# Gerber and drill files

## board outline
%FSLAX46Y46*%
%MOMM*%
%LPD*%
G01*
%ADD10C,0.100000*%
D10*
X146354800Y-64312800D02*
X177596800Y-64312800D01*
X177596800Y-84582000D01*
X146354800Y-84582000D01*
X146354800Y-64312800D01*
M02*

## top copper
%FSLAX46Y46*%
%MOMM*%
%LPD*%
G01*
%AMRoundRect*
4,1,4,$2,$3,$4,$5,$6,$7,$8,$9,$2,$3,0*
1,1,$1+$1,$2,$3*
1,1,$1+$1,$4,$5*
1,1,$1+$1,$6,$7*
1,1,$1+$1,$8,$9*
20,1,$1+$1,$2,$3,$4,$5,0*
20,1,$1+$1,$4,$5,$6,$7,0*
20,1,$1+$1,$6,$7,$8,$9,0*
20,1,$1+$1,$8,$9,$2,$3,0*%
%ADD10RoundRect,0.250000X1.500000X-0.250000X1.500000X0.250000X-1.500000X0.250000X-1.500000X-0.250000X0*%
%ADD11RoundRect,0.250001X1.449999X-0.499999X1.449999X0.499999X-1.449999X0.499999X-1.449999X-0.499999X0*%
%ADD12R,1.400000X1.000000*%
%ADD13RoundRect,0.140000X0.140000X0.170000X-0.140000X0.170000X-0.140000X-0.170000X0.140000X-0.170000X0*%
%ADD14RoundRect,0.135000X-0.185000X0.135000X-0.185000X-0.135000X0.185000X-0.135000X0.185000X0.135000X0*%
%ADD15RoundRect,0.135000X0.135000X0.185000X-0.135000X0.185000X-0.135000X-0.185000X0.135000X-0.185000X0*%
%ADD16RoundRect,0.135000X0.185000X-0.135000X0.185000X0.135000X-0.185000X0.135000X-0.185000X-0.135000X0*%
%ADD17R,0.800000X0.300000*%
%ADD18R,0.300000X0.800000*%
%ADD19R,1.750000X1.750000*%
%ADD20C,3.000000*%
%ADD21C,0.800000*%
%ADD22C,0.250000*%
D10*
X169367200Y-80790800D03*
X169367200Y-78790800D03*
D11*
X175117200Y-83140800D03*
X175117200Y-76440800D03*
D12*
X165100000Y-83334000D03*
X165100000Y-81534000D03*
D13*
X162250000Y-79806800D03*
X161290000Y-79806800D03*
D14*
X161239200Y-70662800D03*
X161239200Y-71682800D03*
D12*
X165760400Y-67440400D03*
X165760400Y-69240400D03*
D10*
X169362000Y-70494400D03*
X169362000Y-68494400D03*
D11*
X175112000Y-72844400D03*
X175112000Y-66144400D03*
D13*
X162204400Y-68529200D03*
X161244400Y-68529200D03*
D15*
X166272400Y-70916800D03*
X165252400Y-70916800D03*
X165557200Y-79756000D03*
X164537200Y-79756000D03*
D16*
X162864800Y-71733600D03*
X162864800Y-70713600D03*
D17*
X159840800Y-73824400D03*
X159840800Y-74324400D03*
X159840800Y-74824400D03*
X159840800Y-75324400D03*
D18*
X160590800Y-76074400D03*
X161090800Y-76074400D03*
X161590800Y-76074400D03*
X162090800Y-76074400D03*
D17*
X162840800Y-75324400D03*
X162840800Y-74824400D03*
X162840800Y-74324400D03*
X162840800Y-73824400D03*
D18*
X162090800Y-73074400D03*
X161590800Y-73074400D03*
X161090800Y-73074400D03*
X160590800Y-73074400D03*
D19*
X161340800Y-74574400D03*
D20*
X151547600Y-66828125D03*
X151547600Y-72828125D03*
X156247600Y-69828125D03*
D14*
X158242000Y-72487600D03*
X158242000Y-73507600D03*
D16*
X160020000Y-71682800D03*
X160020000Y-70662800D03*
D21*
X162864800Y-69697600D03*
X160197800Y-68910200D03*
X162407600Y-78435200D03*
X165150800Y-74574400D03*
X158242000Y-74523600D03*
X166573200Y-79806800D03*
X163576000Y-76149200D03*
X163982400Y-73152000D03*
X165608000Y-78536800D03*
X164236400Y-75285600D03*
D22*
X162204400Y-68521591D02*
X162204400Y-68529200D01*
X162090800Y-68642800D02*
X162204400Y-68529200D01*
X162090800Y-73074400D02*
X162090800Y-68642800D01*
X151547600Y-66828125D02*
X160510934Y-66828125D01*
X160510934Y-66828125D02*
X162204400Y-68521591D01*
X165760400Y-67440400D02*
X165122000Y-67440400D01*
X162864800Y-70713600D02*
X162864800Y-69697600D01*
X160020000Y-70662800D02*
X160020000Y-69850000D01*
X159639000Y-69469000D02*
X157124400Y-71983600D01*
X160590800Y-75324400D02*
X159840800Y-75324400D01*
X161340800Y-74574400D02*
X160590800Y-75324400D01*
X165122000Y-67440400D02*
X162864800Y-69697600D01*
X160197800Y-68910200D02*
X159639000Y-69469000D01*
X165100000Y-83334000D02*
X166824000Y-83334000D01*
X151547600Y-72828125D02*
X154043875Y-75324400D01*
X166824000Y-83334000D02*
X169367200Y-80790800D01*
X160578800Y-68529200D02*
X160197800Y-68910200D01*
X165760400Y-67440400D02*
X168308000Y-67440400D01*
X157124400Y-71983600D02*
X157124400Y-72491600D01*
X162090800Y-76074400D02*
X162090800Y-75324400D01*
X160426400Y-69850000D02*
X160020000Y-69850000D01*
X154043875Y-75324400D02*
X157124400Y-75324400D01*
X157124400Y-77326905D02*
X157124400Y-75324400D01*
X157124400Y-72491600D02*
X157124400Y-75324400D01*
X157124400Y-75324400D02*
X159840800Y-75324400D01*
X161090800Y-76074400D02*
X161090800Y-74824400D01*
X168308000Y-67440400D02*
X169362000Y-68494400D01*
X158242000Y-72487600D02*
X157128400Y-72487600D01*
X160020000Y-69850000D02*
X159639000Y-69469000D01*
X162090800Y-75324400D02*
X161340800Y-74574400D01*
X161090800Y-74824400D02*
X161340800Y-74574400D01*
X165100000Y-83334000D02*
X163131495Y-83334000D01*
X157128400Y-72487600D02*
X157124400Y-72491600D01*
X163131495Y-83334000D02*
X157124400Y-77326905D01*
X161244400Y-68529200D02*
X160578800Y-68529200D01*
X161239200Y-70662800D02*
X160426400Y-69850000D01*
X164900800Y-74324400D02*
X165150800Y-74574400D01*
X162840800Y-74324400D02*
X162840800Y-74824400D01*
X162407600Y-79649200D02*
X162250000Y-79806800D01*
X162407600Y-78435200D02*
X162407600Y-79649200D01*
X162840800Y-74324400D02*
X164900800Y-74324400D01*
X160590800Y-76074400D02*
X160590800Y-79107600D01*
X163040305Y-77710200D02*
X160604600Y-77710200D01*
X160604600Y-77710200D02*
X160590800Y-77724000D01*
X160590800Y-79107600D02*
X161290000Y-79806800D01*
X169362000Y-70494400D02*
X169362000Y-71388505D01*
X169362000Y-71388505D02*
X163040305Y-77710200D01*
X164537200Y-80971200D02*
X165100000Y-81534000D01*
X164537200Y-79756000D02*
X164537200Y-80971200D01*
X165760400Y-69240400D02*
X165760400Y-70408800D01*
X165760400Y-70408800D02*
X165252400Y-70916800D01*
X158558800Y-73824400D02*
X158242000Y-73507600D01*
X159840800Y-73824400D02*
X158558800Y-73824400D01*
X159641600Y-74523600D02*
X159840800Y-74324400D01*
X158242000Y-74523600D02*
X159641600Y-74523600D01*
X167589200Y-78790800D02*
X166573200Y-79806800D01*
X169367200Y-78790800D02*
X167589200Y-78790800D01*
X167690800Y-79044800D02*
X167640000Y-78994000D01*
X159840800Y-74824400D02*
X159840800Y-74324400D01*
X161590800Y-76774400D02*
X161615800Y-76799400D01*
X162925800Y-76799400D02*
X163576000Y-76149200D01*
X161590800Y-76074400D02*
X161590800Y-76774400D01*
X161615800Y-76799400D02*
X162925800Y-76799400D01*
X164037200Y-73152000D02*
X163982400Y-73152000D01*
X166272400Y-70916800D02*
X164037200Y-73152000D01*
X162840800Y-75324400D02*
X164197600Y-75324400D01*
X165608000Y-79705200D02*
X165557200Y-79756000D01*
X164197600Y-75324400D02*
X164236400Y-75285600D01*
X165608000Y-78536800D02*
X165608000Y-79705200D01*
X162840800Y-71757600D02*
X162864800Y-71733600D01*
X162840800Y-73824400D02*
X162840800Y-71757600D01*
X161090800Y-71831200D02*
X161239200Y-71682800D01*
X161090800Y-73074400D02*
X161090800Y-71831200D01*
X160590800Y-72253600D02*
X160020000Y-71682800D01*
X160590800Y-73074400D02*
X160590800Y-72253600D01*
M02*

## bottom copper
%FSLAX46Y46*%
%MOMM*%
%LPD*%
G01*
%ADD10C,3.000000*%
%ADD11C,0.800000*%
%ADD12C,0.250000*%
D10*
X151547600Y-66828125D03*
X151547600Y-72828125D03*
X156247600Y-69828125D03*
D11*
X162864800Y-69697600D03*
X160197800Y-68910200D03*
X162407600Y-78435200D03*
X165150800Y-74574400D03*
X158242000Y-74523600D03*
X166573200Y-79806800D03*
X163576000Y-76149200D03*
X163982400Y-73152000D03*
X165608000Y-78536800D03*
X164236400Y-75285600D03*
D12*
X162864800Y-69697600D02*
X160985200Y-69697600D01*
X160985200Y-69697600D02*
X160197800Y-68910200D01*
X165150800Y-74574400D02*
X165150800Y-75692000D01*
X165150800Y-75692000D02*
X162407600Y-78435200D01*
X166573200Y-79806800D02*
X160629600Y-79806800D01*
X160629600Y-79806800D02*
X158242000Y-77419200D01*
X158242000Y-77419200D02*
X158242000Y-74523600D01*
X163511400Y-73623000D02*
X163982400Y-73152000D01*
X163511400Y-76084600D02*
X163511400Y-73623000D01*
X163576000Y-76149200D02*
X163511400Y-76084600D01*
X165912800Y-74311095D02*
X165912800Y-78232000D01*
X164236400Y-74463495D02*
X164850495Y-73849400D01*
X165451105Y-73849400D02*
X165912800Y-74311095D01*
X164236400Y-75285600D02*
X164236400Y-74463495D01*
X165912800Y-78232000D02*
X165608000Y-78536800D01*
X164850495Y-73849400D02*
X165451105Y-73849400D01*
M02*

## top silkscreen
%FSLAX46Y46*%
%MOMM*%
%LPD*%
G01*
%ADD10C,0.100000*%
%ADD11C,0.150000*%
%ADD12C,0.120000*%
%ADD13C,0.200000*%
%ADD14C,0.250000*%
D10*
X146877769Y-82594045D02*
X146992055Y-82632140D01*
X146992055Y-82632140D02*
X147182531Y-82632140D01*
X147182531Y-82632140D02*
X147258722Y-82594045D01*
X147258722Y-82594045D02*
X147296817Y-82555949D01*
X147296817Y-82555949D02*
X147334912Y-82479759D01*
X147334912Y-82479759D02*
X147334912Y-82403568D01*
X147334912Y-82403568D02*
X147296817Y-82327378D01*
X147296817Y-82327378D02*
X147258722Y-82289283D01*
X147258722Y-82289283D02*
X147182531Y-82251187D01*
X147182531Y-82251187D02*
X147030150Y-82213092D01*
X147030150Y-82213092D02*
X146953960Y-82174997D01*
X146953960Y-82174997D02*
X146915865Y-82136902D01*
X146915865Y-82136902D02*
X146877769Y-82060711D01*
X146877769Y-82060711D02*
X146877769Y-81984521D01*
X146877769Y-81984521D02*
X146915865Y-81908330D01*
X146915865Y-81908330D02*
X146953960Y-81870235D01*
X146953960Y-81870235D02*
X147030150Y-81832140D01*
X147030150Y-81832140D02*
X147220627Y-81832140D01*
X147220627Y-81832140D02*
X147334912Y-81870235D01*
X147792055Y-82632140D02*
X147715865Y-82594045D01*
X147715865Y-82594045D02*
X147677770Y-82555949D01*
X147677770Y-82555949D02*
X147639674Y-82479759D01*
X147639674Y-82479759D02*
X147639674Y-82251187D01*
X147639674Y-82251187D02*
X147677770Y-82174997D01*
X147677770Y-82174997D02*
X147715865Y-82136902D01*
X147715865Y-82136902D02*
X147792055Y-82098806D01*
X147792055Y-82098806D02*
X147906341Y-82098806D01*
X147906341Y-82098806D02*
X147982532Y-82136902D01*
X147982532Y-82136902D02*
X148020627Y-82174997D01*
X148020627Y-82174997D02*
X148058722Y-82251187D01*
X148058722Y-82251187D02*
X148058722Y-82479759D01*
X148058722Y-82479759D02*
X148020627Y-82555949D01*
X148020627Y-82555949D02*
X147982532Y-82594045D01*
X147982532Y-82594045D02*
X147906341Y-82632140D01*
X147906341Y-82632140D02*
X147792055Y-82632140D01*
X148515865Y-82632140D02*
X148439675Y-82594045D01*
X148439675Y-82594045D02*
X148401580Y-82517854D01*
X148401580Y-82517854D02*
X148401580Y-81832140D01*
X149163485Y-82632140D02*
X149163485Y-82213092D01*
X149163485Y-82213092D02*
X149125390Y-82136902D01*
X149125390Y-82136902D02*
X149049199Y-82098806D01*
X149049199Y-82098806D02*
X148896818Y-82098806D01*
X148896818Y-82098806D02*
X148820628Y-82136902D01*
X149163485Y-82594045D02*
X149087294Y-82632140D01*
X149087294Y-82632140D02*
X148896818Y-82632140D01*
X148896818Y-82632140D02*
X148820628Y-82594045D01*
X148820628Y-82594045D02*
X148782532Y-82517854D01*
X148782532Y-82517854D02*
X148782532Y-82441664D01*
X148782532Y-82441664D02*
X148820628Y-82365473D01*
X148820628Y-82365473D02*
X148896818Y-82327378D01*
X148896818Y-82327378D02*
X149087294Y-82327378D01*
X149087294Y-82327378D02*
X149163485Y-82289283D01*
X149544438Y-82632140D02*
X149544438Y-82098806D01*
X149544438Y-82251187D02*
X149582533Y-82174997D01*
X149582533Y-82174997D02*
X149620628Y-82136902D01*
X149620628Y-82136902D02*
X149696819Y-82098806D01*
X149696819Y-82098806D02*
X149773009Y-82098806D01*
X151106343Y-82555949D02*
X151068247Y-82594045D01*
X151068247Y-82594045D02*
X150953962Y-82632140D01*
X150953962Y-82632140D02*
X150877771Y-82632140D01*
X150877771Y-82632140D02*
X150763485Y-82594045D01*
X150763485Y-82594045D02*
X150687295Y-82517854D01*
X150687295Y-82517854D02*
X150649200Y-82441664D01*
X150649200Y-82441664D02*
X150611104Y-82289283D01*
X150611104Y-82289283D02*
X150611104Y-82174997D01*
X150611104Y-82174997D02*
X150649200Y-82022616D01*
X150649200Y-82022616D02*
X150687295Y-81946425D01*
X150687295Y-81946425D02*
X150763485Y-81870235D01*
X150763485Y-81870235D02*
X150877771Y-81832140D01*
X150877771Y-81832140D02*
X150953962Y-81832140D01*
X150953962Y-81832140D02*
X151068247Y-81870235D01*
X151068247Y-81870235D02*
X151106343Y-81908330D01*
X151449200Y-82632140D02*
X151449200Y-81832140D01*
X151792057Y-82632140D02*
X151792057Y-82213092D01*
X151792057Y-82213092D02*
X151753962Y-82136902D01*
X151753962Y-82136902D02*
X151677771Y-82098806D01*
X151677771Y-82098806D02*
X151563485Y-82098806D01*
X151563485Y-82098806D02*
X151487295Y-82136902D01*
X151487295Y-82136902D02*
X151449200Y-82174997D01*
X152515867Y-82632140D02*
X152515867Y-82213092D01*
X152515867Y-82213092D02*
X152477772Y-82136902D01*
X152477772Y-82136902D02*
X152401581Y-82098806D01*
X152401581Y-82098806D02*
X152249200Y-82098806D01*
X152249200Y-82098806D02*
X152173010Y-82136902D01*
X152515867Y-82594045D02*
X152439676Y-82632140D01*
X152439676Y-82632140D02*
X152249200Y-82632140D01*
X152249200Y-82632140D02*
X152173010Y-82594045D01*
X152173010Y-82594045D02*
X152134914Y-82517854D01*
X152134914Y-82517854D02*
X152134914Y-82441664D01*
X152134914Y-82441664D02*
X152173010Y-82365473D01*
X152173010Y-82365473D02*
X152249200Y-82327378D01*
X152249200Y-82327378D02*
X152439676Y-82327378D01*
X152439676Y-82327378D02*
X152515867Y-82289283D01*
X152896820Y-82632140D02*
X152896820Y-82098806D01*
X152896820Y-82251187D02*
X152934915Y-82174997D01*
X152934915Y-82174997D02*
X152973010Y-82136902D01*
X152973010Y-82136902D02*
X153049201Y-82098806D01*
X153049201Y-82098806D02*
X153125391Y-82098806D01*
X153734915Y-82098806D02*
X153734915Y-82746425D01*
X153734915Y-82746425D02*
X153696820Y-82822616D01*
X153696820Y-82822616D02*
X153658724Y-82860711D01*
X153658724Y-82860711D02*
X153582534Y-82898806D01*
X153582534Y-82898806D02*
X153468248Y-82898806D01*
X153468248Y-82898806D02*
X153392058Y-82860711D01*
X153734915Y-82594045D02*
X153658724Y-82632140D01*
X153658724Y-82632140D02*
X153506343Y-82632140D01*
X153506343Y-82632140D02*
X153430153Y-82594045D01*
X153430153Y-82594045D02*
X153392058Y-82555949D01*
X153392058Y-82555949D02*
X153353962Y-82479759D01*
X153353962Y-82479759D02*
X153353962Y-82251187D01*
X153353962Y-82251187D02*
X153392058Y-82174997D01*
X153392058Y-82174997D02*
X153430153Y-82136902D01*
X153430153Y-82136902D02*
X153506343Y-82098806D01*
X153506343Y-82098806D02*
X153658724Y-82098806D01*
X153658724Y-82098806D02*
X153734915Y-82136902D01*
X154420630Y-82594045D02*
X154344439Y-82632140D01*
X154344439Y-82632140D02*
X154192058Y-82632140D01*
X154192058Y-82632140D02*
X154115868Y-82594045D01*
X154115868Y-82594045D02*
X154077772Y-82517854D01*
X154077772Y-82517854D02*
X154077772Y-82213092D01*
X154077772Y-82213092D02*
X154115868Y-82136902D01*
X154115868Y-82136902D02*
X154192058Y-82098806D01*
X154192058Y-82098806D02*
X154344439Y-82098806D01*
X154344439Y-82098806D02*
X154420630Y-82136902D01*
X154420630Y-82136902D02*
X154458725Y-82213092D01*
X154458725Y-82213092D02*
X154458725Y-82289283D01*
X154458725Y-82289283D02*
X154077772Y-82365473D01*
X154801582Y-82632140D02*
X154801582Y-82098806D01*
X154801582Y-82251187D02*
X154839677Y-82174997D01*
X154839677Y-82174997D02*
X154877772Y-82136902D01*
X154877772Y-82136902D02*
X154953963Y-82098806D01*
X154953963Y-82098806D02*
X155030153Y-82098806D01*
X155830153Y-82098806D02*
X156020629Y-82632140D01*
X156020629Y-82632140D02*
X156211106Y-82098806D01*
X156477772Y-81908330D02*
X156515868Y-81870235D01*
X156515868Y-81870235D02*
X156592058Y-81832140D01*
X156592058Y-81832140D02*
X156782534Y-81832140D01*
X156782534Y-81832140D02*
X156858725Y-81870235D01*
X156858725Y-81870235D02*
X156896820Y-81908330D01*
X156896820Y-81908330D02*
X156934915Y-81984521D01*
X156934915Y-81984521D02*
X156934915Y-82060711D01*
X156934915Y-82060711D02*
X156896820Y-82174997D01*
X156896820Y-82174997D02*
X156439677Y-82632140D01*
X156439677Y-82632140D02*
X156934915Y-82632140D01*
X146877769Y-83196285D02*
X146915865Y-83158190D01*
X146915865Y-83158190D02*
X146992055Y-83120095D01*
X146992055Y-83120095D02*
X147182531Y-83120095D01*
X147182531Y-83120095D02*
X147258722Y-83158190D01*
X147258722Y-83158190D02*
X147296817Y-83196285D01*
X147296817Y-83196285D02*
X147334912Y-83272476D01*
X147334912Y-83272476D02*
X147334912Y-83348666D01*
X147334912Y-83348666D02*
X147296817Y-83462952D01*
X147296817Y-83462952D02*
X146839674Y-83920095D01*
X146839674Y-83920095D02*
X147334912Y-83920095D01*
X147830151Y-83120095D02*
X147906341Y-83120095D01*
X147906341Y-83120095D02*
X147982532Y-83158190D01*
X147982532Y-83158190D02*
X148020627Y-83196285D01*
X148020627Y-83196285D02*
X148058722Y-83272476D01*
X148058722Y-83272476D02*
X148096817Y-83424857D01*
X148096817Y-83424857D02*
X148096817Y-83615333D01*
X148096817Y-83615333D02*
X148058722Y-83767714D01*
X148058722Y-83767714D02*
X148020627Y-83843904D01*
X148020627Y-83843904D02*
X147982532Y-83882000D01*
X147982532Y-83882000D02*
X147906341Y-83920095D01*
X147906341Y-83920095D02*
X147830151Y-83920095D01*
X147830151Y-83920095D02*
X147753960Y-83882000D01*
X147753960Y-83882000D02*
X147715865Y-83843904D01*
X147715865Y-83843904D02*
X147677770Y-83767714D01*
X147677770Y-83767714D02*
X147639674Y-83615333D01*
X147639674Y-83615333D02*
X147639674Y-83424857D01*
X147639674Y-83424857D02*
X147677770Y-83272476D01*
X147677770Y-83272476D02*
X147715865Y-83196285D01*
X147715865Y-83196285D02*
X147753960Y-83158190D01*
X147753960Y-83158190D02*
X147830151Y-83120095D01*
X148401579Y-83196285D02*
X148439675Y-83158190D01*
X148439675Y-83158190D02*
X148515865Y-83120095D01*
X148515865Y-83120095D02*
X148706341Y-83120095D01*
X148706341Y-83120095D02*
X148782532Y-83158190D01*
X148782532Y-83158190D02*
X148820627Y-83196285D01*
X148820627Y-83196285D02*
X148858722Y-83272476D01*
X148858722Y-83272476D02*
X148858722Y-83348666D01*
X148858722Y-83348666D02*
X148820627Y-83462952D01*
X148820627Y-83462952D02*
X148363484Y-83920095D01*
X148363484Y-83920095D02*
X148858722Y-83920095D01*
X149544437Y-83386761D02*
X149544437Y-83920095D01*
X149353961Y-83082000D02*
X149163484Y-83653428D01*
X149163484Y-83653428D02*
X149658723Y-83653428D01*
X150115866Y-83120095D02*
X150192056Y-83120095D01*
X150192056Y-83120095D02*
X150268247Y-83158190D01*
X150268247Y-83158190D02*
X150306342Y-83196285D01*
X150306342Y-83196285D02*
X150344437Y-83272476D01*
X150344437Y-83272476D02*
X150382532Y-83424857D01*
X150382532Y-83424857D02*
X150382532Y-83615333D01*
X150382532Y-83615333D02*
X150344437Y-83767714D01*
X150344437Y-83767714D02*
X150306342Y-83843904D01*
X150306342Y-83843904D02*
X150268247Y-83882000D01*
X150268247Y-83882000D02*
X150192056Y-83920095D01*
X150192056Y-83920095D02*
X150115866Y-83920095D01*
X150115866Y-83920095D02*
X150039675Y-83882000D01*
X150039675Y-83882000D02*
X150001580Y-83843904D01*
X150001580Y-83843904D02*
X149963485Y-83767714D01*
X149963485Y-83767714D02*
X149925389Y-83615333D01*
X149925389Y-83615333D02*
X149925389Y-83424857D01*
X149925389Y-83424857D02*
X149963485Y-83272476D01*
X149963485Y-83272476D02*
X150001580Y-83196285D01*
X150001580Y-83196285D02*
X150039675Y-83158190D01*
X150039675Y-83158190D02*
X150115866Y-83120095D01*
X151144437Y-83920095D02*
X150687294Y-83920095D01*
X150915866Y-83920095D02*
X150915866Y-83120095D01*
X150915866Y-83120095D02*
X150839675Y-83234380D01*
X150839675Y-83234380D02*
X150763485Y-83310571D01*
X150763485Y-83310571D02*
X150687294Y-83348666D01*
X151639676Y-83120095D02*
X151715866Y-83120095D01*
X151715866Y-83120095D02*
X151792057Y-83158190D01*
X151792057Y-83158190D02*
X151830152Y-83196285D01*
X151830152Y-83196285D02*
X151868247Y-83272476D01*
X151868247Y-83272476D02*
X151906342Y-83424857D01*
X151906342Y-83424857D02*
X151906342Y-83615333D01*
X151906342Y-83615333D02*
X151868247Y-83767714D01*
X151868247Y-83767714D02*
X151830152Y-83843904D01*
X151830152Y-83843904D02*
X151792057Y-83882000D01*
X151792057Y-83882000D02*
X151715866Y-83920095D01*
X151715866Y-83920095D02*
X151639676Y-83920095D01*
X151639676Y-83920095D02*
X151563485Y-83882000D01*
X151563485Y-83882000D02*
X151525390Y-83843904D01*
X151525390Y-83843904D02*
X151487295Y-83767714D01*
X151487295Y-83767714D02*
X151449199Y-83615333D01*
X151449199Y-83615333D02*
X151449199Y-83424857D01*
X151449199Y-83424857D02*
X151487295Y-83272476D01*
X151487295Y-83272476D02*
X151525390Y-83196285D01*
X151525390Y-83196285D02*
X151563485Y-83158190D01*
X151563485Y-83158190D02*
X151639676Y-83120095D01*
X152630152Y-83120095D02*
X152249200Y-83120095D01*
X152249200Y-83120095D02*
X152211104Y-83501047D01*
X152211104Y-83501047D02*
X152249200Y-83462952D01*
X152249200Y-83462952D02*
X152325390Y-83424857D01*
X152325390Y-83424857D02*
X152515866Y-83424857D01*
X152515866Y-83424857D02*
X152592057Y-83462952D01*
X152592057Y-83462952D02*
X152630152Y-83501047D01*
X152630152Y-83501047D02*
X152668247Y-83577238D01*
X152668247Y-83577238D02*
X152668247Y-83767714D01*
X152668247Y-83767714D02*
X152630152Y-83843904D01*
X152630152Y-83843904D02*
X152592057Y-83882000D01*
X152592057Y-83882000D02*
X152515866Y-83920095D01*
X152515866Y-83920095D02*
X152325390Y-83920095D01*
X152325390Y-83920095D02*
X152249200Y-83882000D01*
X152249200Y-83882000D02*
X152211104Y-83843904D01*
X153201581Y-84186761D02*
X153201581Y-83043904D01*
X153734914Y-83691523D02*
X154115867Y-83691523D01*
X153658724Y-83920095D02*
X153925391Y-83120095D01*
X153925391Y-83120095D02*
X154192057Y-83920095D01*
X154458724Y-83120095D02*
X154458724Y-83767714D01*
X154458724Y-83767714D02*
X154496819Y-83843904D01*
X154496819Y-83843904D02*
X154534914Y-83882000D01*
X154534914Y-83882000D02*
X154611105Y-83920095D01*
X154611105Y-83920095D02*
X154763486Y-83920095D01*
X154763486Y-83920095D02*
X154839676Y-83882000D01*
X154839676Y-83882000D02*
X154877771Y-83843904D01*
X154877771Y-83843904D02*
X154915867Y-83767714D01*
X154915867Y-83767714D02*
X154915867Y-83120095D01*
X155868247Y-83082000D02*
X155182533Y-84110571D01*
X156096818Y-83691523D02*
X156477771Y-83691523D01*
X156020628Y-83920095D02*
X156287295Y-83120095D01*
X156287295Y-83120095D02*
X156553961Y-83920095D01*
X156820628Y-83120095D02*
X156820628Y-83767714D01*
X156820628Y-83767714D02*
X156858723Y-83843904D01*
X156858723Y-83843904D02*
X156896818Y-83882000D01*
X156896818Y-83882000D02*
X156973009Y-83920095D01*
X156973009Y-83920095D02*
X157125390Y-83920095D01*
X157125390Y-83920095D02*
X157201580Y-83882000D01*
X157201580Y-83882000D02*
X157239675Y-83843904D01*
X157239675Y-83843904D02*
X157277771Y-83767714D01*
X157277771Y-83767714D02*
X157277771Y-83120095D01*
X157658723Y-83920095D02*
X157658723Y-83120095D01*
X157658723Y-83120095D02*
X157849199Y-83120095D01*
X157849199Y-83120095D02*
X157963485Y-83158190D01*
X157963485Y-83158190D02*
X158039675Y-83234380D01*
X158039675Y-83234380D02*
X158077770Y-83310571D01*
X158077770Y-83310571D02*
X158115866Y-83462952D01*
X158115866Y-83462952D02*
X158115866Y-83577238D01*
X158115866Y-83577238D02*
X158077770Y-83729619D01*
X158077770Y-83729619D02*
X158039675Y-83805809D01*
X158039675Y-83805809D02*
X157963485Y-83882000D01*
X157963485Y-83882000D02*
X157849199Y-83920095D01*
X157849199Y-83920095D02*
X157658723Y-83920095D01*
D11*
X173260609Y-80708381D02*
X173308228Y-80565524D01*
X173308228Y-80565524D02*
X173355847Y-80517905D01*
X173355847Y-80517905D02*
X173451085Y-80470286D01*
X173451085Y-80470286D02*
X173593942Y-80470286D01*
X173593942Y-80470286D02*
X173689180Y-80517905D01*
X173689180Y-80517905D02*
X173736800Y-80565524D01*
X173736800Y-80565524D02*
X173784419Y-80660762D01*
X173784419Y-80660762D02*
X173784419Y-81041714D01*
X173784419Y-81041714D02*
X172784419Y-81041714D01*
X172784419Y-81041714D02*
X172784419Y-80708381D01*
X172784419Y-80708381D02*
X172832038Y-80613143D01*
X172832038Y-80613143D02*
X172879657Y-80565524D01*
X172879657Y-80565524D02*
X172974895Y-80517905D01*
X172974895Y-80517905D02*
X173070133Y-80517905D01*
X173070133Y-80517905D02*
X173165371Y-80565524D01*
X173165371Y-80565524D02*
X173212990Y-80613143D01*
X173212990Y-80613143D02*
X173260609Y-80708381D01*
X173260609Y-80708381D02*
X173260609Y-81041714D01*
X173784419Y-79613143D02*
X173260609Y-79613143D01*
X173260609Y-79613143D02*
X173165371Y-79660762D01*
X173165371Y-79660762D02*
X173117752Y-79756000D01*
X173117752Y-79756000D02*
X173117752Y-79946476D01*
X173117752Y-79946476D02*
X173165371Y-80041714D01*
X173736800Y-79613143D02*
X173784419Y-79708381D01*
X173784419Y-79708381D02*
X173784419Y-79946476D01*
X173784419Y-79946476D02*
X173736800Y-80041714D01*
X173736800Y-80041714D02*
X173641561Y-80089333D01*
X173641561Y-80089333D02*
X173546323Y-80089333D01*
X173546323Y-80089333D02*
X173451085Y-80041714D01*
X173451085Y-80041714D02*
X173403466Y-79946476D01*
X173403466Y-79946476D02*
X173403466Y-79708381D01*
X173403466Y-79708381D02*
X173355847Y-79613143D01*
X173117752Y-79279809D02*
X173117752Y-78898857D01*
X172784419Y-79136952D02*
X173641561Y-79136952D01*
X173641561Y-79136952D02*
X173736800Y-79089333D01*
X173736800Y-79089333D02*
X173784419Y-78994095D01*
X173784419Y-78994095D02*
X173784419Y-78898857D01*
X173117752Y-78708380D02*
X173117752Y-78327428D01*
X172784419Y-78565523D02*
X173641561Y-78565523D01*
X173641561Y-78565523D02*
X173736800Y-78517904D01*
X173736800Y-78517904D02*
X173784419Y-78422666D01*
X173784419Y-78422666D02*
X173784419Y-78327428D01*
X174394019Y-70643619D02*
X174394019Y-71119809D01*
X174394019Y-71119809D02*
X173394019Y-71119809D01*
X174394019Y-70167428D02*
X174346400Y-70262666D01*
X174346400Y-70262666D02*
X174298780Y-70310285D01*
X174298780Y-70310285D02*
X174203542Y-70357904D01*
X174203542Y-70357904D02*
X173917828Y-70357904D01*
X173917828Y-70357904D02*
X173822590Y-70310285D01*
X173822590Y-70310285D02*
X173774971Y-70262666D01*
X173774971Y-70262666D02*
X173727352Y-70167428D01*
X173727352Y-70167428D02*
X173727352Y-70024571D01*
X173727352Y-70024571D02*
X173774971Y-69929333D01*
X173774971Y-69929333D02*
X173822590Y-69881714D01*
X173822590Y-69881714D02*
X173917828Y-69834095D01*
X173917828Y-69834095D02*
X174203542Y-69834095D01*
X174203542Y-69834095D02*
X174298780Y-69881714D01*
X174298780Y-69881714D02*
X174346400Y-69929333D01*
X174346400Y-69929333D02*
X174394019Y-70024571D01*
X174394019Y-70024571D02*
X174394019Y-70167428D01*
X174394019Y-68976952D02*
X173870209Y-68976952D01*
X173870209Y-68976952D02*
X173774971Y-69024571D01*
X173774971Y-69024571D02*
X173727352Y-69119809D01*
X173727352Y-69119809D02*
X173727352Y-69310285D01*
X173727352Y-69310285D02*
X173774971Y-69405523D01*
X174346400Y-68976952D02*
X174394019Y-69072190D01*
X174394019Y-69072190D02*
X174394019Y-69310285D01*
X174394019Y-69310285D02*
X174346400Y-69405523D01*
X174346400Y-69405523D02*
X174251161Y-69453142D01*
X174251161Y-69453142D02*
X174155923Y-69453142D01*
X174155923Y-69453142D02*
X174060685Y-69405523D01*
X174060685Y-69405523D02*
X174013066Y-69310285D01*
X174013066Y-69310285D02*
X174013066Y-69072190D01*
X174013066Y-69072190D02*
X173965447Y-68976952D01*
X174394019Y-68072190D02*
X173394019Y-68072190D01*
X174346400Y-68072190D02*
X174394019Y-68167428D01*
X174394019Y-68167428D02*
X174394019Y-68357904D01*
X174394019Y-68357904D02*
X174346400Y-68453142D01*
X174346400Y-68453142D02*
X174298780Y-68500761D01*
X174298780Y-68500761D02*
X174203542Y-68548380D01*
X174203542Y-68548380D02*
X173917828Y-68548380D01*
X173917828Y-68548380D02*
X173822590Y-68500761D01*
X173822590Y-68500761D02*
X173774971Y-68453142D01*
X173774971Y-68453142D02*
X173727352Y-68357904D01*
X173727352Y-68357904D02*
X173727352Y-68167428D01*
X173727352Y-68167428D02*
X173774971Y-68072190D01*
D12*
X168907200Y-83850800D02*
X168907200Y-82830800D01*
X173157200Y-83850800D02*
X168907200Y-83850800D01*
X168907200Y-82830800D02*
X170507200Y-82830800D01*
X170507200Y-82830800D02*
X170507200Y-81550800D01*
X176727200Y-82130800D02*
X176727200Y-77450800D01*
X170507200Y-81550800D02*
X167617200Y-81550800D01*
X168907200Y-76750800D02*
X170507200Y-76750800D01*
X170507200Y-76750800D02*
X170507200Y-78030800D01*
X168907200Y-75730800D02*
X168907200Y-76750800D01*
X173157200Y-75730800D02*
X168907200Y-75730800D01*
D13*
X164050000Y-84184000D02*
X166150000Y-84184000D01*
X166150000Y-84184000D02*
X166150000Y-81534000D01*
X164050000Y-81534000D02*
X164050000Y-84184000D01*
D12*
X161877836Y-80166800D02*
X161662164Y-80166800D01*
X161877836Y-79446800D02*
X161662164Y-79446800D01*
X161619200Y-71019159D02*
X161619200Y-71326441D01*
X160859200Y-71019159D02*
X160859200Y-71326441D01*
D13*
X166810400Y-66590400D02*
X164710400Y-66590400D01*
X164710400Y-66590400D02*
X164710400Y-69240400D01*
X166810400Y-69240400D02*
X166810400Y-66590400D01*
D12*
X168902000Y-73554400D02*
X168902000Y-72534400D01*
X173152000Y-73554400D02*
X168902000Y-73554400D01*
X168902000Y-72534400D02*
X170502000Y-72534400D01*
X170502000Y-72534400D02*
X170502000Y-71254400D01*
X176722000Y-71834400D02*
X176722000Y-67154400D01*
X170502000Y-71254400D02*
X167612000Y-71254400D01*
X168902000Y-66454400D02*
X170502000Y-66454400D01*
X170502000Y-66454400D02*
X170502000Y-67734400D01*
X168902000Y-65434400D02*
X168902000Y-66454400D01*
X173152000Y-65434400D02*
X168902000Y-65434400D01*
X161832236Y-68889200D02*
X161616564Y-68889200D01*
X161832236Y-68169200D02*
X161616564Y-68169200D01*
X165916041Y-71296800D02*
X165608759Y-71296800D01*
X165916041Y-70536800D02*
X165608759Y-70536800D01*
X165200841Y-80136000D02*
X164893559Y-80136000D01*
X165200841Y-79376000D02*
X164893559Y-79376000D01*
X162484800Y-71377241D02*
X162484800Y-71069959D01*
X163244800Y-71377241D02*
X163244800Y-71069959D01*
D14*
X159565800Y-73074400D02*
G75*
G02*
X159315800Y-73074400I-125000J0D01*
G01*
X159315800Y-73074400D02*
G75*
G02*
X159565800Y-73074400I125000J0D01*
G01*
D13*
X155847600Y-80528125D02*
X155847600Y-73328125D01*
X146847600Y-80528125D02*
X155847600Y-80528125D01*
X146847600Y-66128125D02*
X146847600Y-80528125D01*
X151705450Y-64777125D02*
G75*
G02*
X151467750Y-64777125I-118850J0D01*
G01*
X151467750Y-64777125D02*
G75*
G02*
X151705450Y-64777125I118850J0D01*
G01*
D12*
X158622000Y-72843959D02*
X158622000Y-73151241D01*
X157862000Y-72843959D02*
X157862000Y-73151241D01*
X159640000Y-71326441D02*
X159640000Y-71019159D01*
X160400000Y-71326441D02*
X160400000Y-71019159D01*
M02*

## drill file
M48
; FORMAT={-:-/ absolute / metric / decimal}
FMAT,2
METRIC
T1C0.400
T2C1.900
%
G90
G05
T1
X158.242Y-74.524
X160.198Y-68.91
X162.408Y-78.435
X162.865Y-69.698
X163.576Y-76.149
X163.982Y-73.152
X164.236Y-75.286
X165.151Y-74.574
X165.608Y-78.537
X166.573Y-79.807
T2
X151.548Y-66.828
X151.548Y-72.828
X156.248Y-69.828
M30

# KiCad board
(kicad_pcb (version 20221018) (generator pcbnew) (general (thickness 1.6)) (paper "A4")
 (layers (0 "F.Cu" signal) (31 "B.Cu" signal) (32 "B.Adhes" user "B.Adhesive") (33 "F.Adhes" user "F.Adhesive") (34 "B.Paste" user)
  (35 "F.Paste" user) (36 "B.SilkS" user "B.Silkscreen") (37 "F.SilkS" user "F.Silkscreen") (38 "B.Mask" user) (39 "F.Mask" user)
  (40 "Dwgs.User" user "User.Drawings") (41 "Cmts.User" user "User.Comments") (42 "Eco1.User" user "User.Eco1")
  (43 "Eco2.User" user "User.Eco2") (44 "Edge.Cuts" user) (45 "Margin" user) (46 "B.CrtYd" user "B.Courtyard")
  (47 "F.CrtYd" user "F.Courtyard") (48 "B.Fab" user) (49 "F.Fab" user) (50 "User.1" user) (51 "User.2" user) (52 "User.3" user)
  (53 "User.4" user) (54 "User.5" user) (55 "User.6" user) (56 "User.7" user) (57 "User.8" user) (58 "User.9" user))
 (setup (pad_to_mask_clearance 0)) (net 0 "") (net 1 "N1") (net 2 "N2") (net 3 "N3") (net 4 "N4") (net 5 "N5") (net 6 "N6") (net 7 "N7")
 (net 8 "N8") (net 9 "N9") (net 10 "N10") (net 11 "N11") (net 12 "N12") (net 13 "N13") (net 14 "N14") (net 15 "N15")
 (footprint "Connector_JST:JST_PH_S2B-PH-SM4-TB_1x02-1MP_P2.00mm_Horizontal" (layer "F.Cu") (at 172.2172 79.7908 90)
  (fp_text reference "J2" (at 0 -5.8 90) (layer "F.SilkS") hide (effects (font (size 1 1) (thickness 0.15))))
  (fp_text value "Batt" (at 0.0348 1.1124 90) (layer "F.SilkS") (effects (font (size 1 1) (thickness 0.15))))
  (fp_line (start -4.06 -3.31) (end -3.04 -3.31) (stroke (width 0.12) (type solid)) (layer "F.SilkS"))
  (fp_line (start -4.06 0.94) (end -4.06 -3.31) (stroke (width 0.12) (type solid)) (layer "F.SilkS"))
  (fp_line (start -3.04 -3.31) (end -3.04 -1.71) (stroke (width 0.12) (type solid)) (layer "F.SilkS"))
  (fp_line (start -3.04 -1.71) (end -1.76 -1.71) (stroke (width 0.12) (type solid)) (layer "F.SilkS"))
  (fp_line (start -2.34 4.51) (end 2.34 4.51) (stroke (width 0.12) (type solid)) (layer "F.SilkS"))
  (fp_line (start -1.76 -1.71) (end -1.76 -4.6) (stroke (width 0.12) (type solid)) (layer "F.SilkS"))
  (fp_line (start 3.04 -3.31) (end 3.04 -1.71) (stroke (width 0.12) (type solid)) (layer "F.SilkS"))
  (fp_line (start 3.04 -1.71) (end 1.76 -1.71) (stroke (width 0.12) (type solid)) (layer "F.SilkS"))
  (fp_line (start 4.06 -3.31) (end 3.04 -3.31) (stroke (width 0.12) (type solid)) (layer "F.SilkS"))
  (fp_line (start 4.06 0.94) (end 4.06 -3.31) (stroke (width 0.12) (type solid)) (layer "F.SilkS"))
  (pad "1" smd roundrect (at -1 -2.85 90) (size 1 3.5) (layers "F.Cu" "F.Paste" "F.Mask") (roundrect_rratio 0.25) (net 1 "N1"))
  (pad "2" smd roundrect (at 1 -2.85 90) (size 1 3.5) (layers "F.Cu" "F.Paste" "F.Mask") (roundrect_rratio 0.25) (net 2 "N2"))
  (pad "MP" smd roundrect (at -3.35 2.9 90) (size 1.5 3.4) (layers "F.Cu" "F.Paste" "F.Mask") (roundrect_rratio 0.1666673333))
  (pad "MP" smd roundrect (at 3.35 2.9 90) (size 1.5 3.4) (layers "F.Cu" "F.Paste" "F.Mask") (roundrect_rratio 0.1666673333)))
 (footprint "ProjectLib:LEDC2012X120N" (layer "F.Cu") (at 165.1 82.434 90)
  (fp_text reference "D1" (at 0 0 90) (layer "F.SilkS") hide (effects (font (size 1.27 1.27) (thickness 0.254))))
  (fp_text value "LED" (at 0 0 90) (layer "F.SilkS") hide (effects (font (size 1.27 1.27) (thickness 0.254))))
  (fp_line (start -1.75 -1.05) (end -1.75 1.05) (stroke (width 0.2) (type solid)) (layer "F.SilkS"))
  (fp_line (start -1.75 1.05) (end 0.9 1.05) (stroke (width 0.2) (type solid)) (layer "F.SilkS"))
  (fp_line (start 0.9 -1.05) (end -1.75 -1.05) (stroke (width 0.2) (type solid)) (layer "F.SilkS"))
  (pad "1" smd rect (at -0.9 0 90) (size 1 1.4) (layers "F.Cu" "F.Paste" "F.Mask") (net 1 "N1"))
  (pad "2" smd rect (at 0.9 0 90) (size 1 1.4) (layers "F.Cu" "F.Paste" "F.Mask") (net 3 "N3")))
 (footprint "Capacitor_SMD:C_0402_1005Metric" (layer "F.Cu") (at 161.77 79.8068 180)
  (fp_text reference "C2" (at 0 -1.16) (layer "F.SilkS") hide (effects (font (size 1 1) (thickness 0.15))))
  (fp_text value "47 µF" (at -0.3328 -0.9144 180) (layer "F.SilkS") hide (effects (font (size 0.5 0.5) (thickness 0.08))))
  (fp_line (start -0.107836 -0.36) (end 0.107836 -0.36) (stroke (width 0.12) (type solid)) (layer "F.SilkS"))
  (fp_line (start -0.107836 0.36) (end 0.107836 0.36) (stroke (width 0.12) (type solid)) (layer "F.SilkS"))
  (pad "1" smd roundrect (at -0.48 0 180) (size 0.56 0.62) (layers "F.Cu" "F.Paste" "F.Mask") (roundrect_rratio 0.25) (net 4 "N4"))
  (pad "2" smd roundrect (at 0.48 0 180) (size 0.56 0.62) (layers "F.Cu" "F.Paste" "F.Mask") (roundrect_rratio 0.25) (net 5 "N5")))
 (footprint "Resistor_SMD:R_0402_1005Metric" (layer "F.Cu") (at 161.2392 71.1728 -90)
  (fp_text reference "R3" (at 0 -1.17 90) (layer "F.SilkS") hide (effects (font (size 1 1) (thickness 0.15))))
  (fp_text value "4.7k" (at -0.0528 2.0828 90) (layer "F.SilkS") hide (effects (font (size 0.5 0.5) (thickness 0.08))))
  (fp_line (start -0.153641 -0.38) (end 0.153641 -0.38) (stroke (width 0.12) (type solid)) (layer "F.SilkS"))
  (fp_line (start -0.153641 0.38) (end 0.153641 0.38) (stroke (width 0.12) (type solid)) (layer "F.SilkS"))
  (pad "1" smd roundrect (at -0.51 0 270) (size 0.54 0.64) (layers "F.Cu" "F.Paste" "F.Mask") (roundrect_rratio 0.25) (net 1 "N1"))
  (pad "2" smd roundrect (at 0.51 0 270) (size 0.54 0.64) (layers "F.Cu" "F.Paste" "F.Mask") (roundrect_rratio 0.25) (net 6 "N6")))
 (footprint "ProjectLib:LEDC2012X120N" (layer "F.Cu") (at 165.7604 68.3404 -90)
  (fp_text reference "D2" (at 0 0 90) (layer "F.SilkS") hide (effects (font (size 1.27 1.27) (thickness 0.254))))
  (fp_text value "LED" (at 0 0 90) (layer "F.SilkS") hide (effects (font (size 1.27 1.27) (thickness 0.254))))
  (fp_line (start -1.75 -1.05) (end -1.75 1.05) (stroke (width 0.2) (type solid)) (layer "F.SilkS"))
  (fp_line (start -1.75 1.05) (end 0.9 1.05) (stroke (width 0.2) (type solid)) (layer "F.SilkS"))
  (fp_line (start 0.9 -1.05) (end -1.75 -1.05) (stroke (width 0.2) (type solid)) (layer "F.SilkS"))
  (pad "1" smd rect (at -0.9 0 270) (size 1 1.4) (layers "F.Cu" "F.Paste" "F.Mask") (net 1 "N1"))
  (pad "2" smd rect (at 0.9 0 270) (size 1 1.4) (layers "F.Cu" "F.Paste" "F.Mask") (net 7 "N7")))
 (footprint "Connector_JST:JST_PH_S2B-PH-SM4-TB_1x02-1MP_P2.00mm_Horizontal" (layer "F.Cu") (at 172.212 69.4944 90)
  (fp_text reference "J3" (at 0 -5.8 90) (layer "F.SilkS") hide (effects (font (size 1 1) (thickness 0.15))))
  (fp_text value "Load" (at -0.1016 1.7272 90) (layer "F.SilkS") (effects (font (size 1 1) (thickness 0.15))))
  (fp_line (start -4.06 -3.31) (end -3.04 -3.31) (stroke (width 0.12) (type solid)) (layer "F.SilkS"))
  (fp_line (start -4.06 0.94) (end -4.06 -3.31) (stroke (width 0.12) (type solid)) (layer "F.SilkS"))
  (fp_line (start -3.04 -3.31) (end -3.04 -1.71) (stroke (width 0.12) (type solid)) (layer "F.SilkS"))
  (fp_line (start -3.04 -1.71) (end -1.76 -1.71) (stroke (width 0.12) (type solid)) (layer "F.SilkS"))
  (fp_line (start -2.34 4.51) (end 2.34 4.51) (stroke (width 0.12) (type solid)) (layer "F.SilkS"))
  (fp_line (start -1.76 -1.71) (end -1.76 -4.6) (stroke (width 0.12) (type solid)) (layer "F.SilkS"))
  (fp_line (start 3.04 -3.31) (end 3.04 -1.71) (stroke (width 0.12) (type solid)) (layer "F.SilkS"))
  (fp_line (start 3.04 -1.71) (end 1.76 -1.71) (stroke (width 0.12) (type solid)) (layer "F.SilkS"))
  (fp_line (start 4.06 -3.31) (end 3.04 -3.31) (stroke (width 0.12) (type solid)) (layer "F.SilkS"))
  (fp_line (start 4.06 0.94) (end 4.06 -3.31) (stroke (width 0.12) (type solid)) (layer "F.SilkS"))
  (pad "1" smd roundrect (at -1 -2.85 90) (size 1 3.5) (layers "F.Cu" "F.Paste" "F.Mask") (roundrect_rratio 0.25) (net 5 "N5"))
  (pad "2" smd roundrect (at 1 -2.85 90) (size 1 3.5) (layers "F.Cu" "F.Paste" "F.Mask") (roundrect_rratio 0.25) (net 1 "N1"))
  (pad "MP" smd roundrect (at -3.35 2.9 90) (size 1.5 3.4) (layers "F.Cu" "F.Paste" "F.Mask") (roundrect_rratio 0.1666673333))
  (pad "MP" smd roundrect (at 3.35 2.9 90) (size 1.5 3.4) (layers "F.Cu" "F.Paste" "F.Mask") (roundrect_rratio 0.1666673333)))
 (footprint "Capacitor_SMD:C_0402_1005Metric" (layer "F.Cu") (at 161.7244 68.5292 180)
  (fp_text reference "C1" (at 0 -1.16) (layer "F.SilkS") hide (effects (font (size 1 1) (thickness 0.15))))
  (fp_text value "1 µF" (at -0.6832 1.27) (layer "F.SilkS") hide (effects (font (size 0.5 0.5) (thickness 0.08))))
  (fp_line (start -0.107836 -0.36) (end 0.107836 -0.36) (stroke (width 0.12) (type solid)) (layer "F.SilkS"))
  (fp_line (start -0.107836 0.36) (end 0.107836 0.36) (stroke (width 0.12) (type solid)) (layer "F.SilkS"))
  (pad "1" smd roundrect (at -0.48 0 180) (size 0.56 0.62) (layers "F.Cu" "F.Paste" "F.Mask") (roundrect_rratio 0.25) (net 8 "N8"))
  (pad "2" smd roundrect (at 0.48 0 180) (size 0.56 0.62) (layers "F.Cu" "F.Paste" "F.Mask") (roundrect_rratio 0.25) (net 1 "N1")))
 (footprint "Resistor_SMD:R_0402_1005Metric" (layer "F.Cu") (at 165.7624 70.9168 180)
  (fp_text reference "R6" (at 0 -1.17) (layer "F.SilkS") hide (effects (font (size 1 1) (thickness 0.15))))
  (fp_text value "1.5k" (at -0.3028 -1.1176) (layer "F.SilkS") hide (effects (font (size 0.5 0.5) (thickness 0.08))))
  (fp_line (start -0.153641 -0.38) (end 0.153641 -0.38) (stroke (width 0.12) (type solid)) (layer "F.SilkS"))
  (fp_line (start -0.153641 0.38) (end 0.153641 0.38) (stroke (width 0.12) (type solid)) (layer "F.SilkS"))
  (pad "1" smd roundrect (at -0.51 0 180) (size 0.54 0.64) (layers "F.Cu" "F.Paste" "F.Mask") (roundrect_rratio 0.25) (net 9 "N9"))
  (pad "2" smd roundrect (at 0.51 0 180) (size 0.54 0.64) (layers "F.Cu" "F.Paste" "F.Mask") (roundrect_rratio 0.25) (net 7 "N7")))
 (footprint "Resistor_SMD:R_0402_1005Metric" (layer "F.Cu") (at 165.0472 79.756 180)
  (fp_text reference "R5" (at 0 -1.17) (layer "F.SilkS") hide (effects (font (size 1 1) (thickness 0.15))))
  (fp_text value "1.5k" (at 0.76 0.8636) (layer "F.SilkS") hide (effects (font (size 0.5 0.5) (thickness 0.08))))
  (fp_line (start -0.153641 -0.38) (end 0.153641 -0.38) (stroke (width 0.12) (type solid)) (layer "F.SilkS"))
  (fp_line (start -0.153641 0.38) (end 0.153641 0.38) (stroke (width 0.12) (type solid)) (layer "F.SilkS"))
  (pad "1" smd roundrect (at -0.51 0 180) (size 0.54 0.64) (layers "F.Cu" "F.Paste" "F.Mask") (roundrect_rratio 0.25) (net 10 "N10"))
  (pad "2" smd roundrect (at 0.51 0 180) (size 0.54 0.64) (layers "F.Cu" "F.Paste" "F.Mask") (roundrect_rratio 0.25) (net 3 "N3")))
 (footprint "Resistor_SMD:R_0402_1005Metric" (layer "F.Cu") (at 162.8648 71.2236 90)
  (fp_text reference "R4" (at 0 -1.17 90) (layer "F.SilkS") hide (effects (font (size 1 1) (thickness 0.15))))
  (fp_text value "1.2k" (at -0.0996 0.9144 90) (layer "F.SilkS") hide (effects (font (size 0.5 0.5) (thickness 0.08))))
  (fp_line (start -0.153641 -0.38) (end 0.153641 -0.38) (stroke (width 0.12) (type solid)) (layer "F.SilkS"))
  (fp_line (start -0.153641 0.38) (end 0.153641 0.38) (stroke (width 0.12) (type solid)) (layer "F.SilkS"))
  (pad "1" smd roundrect (at -0.51 0 90) (size 0.54 0.64) (layers "F.Cu" "F.Paste" "F.Mask") (roundrect_rratio 0.25) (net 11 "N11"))
  (pad "2" smd roundrect (at 0.51 0 90) (size 0.54 0.64) (layers "F.Cu" "F.Paste" "F.Mask") (roundrect_rratio 0.25) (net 1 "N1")))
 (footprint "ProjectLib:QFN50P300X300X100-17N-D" (layer "F.Cu") (at 161.3408 74.5744)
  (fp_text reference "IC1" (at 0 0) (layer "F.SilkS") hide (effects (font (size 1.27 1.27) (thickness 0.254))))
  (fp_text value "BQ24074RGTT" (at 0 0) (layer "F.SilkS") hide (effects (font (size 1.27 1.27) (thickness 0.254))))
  (fp_circle (center -1.9 -1.5) (end -1.9 -1.375) (stroke (width 0.25) (type solid)) (fill none) (layer "F.SilkS"))
  (pad "1" smd rect (at -1.5 -0.75 90) (size 0.3 0.8) (layers "F.Cu" "F.Paste" "F.Mask") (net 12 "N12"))
  (pad "2" smd rect (at -1.5 -0.25 90) (size 0.3 0.8) (layers "F.Cu" "F.Paste" "F.Mask") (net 2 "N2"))
  (pad "3" smd rect (at -1.5 0.25 90) (size 0.3 0.8) (layers "F.Cu" "F.Paste" "F.Mask") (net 2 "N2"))
  (pad "4" smd rect (at -1.5 0.75 90) (size 0.3 0.8) (layers "F.Cu" "F.Paste" "F.Mask") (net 1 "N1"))
  (pad "5" smd rect (at -0.75 1.5) (size 0.3 0.8) (layers "F.Cu" "F.Paste" "F.Mask") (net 5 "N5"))
  (pad "6" smd rect (at -0.25 1.5) (size 0.3 0.8) (layers "F.Cu" "F.Paste" "F.Mask") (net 1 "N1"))
  (pad "7" smd rect (at 0.25 1.5) (size 0.3 0.8) (layers "F.Cu" "F.Paste" "F.Mask") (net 9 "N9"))
  (pad "8" smd rect (at 0.75 1.5) (size 0.3 0.8) (layers "F.Cu" "F.Paste" "F.Mask") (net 1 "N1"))
  (pad "9" smd rect (at 1.5 0.75 90) (size 0.3 0.8) (layers "F.Cu" "F.Paste" "F.Mask") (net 10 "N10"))
  (pad "10" smd rect (at 1.5 0.25 90) (size 0.3 0.8) (layers "F.Cu" "F.Paste" "F.Mask") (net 4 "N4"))
  (pad "11" smd rect (at 1.5 -0.25 90) (size 0.3 0.8) (layers "F.Cu" "F.Paste" "F.Mask") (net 4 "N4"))
  (pad "12" smd rect (at 1.5 -0.75 90) (size 0.3 0.8) (layers "F.Cu" "F.Paste" "F.Mask") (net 11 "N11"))
  (pad "13" smd rect (at 0.75 -1.5) (size 0.3 0.8) (layers "F.Cu" "F.Paste" "F.Mask") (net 8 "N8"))
  (pad "14" smd rect (at 0.25 -1.5) (size 0.3 0.8) (layers "F.Cu" "F.Paste" "F.Mask") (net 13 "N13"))
  (pad "15" smd rect (at -0.25 -1.5) (size 0.3 0.8) (layers "F.Cu" "F.Paste" "F.Mask") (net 6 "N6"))
  (pad "16" smd rect (at -0.75 -1.5) (size 0.3 0.8) (layers "F.Cu" "F.Paste" "F.Mask") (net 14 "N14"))
  (pad "17" smd rect (at 0 0) (size 1.75 1.75) (layers "F.Cu" "F.Paste" "F.Mask") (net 1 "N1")))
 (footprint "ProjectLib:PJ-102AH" (layer "F.Cu") (at 155.8476 69.828125 180)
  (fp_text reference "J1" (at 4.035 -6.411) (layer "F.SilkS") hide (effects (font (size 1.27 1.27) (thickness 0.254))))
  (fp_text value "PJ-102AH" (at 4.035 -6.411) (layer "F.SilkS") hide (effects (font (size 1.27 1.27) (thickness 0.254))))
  (fp_line (start 0 -10.7) (end 0 -3.5) (stroke (width 0.2) (type solid)) (layer "F.SilkS"))
  (fp_line (start 9 -10.7) (end 0 -10.7) (stroke (width 0.2) (type solid)) (layer "F.SilkS"))
  (fp_line (start 9 3.7) (end 9 -10.7) (stroke (width 0.2) (type solid)) (layer "F.SilkS"))
  (fp_circle (center 4.261 5.051) (end 4.261 5.16985) (stroke (width 0.2) (type solid)) (fill none) (layer "F.SilkS"))
  (pad "1" thru_hole circle (at 4.3 3 180) (size 3 3) (drill 1.9) (layers "*.Cu" "*.Mask") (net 8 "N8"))
  (pad "2" thru_hole circle (at 4.3 -3 180) (size 3 3) (drill 1.9) (layers "*.Cu" "*.Mask") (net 1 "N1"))
  (pad "3" thru_hole circle (at -0.4 0 180) (size 3 3) (drill 1.9) (layers "*.Cu" "*.Mask") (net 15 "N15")))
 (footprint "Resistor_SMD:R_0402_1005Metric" (layer "F.Cu") (at 158.242 72.9976 -90)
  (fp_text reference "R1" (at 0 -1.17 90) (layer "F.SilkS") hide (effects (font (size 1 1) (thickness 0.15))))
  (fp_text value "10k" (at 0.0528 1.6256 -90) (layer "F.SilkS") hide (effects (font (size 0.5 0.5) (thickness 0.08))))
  (fp_line (start -0.153641 -0.38) (end 0.153641 -0.38) (stroke (width 0.12) (type solid)) (layer "F.SilkS"))
  (fp_line (start -0.153641 0.38) (end 0.153641 0.38) (stroke (width 0.12) (type solid)) (layer "F.SilkS"))
  (pad "1" smd roundrect (at -0.51 0 270) (size 0.54 0.64) (layers "F.Cu" "F.Paste" "F.Mask") (roundrect_rratio 0.25) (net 1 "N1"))
  (pad "2" smd roundrect (at 0.51 0 270) (size 0.54 0.64) (layers "F.Cu" "F.Paste" "F.Mask") (roundrect_rratio 0.25) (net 12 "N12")))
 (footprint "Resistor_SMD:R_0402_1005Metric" (layer "F.Cu") (at 160.02 71.1728 90)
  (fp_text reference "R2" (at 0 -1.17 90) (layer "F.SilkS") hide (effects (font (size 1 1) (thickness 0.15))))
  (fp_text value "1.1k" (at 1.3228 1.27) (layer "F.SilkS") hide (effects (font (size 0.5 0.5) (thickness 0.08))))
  (fp_line (start -0.153641 -0.38) (end 0.153641 -0.38) (stroke (width 0.12) (type solid)) (layer "F.SilkS"))
  (fp_line (start -0.153641 0.38) (end 0.153641 0.38) (stroke (width 0.12) (type solid)) (layer "F.SilkS"))
  (pad "1" smd roundrect (at -0.51 0 90) (size 0.54 0.64) (layers "F.Cu" "F.Paste" "F.Mask") (roundrect_rratio 0.25) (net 14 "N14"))
  (pad "2" smd roundrect (at 0.51 0 90) (size 0.54 0.64) (layers "F.Cu" "F.Paste" "F.Mask") (roundrect_rratio 0.25) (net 1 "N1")))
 (gr_rect (start 146.3548 64.3128) (end 177.5968 84.582) (stroke (width 0.1) (type default)) (fill none) (layer "Edge.Cuts"))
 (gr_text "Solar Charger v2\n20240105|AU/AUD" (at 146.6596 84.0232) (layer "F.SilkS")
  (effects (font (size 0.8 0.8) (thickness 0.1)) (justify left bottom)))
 (segment (start 162.2044 68.521591) (end 162.2044 68.5292) (width 0.25) (layer "F.Cu") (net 8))
 (segment (start 162.0908 68.6428) (end 162.2044 68.5292) (width 0.25) (layer "F.Cu") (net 8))
 (segment (start 162.0908 73.0744) (end 162.0908 68.6428) (width 0.25) (layer "F.Cu") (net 8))
 (segment (start 151.5476 66.828125) (end 160.510934 66.828125) (width 0.25) (layer "F.Cu") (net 8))
 (segment (start 160.510934 66.828125) (end 162.2044 68.521591) (width 0.25) (layer "F.Cu") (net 8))
 (segment (start 165.7604 67.4404) (end 165.122 67.4404) (width 0.25) (layer "F.Cu") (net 1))
 (segment (start 162.8648 70.7136) (end 162.8648 69.6976) (width 0.25) (layer "F.Cu") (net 1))
 (segment (start 160.02 70.6628) (end 160.02 69.85) (width 0.25) (layer "F.Cu") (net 1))
 (segment (start 159.639 69.469) (end 157.1244 71.9836) (width 0.25) (layer "F.Cu") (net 1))
 (segment (start 160.5908 75.3244) (end 159.8408 75.3244) (width 0.25) (layer "F.Cu") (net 1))
 (segment (start 161.3408 74.5744) (end 160.5908 75.3244) (width 0.25) (layer "F.Cu") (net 1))
 (segment (start 165.122 67.4404) (end 162.8648 69.6976) (width 0.25) (layer "F.Cu") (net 1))
 (segment (start 160.1978 68.9102) (end 159.639 69.469) (width 0.25) (layer "F.Cu") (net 1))
 (segment (start 165.1 83.334) (end 166.824 83.334) (width 0.25) (layer "F.Cu") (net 1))
 (segment (start 151.5476 72.828125) (end 154.043875 75.3244) (width 0.25) (layer "F.Cu") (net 1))
 (segment (start 166.824 83.334) (end 169.3672 80.7908) (width 0.25) (layer "F.Cu") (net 1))
 (segment (start 160.5788 68.5292) (end 160.1978 68.9102) (width 0.25) (layer "F.Cu") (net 1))
 (segment (start 165.7604 67.4404) (end 168.308 67.4404) (width 0.25) (layer "F.Cu") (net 1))
 (segment (start 157.1244 71.9836) (end 157.1244 72.4916) (width 0.25) (layer "F.Cu") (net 1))
 (segment (start 162.0908 76.0744) (end 162.0908 75.3244) (width 0.25) (layer "F.Cu") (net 1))
 (segment (start 160.4264 69.85) (end 160.02 69.85) (width 0.25) (layer "F.Cu") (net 1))
 (segment (start 154.043875 75.3244) (end 157.1244 75.3244) (width 0.25) (layer "F.Cu") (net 1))
 (segment (start 157.1244 77.326905) (end 157.1244 75.3244) (width 0.25) (layer "F.Cu") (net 1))
 (segment (start 157.1244 72.4916) (end 157.1244 75.3244) (width 0.25) (layer "F.Cu") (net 1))
 (segment (start 157.1244 75.3244) (end 159.8408 75.3244) (width 0.25) (layer "F.Cu") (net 1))
 (segment (start 161.0908 76.0744) (end 161.0908 74.8244) (width 0.25) (layer "F.Cu") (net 1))
 (segment (start 168.308 67.4404) (end 169.362 68.4944) (width 0.25) (layer "F.Cu") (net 1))
 (segment (start 158.242 72.4876) (end 157.1284 72.4876) (width 0.25) (layer "F.Cu") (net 1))
 (segment (start 160.02 69.85) (end 159.639 69.469) (width 0.25) (layer "F.Cu") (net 1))
 (segment (start 162.0908 75.3244) (end 161.3408 74.5744) (width 0.25) (layer "F.Cu") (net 1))
 (segment (start 161.0908 74.8244) (end 161.3408 74.5744) (width 0.25) (layer "F.Cu") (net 1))
 (segment (start 165.1 83.334) (end 163.131495 83.334) (width 0.25) (layer "F.Cu") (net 1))
 (segment (start 157.1284 72.4876) (end 157.1244 72.4916) (width 0.25) (layer "F.Cu") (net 1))
 (segment (start 163.131495 83.334) (end 157.1244 77.326905) (width 0.25) (layer "F.Cu") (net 1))
 (segment (start 161.2444 68.5292) (end 160.5788 68.5292) (width 0.25) (layer "F.Cu") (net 1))
 (segment (start 161.2392 70.6628) (end 160.4264 69.85) (width 0.25) (layer "F.Cu") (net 1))
 (via (at 162.8648 69.6976) (size 0.8) (drill 0.4) (layers "F.Cu" "B.Cu") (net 1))
 (via (at 160.1978 68.9102) (size 0.8) (drill 0.4) (layers "F.Cu" "B.Cu") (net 1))
 (segment (start 162.8648 69.6976) (end 160.9852 69.6976) (width 0.25) (layer "B.Cu") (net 1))
 (segment (start 160.9852 69.6976) (end 160.1978 68.9102) (width 0.25) (layer "B.Cu") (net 1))
 (segment (start 164.9008 74.3244) (end 165.1508 74.5744) (width 0.25) (layer "F.Cu") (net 4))
 (segment (start 162.8408 74.3244) (end 162.8408 74.8244) (width 0.25) (layer "F.Cu") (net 4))
 (segment (start 162.4076 79.6492) (end 162.25 79.8068) (width 0.25) (layer "F.Cu") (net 4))
 (segment (start 162.4076 78.4352) (end 162.4076 79.6492) (width 0.25) (layer "F.Cu") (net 4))
 (segment (start 162.8408 74.3244) (end 164.9008 74.3244) (width 0.25) (layer "F.Cu") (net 4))
 (via (at 162.4076 78.4352) (size 0.8) (drill 0.4) (layers "F.Cu" "B.Cu") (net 4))
 (via (at 165.1508 74.5744) (size 0.8) (drill 0.4) (layers "F.Cu" "B.Cu") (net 4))
 (segment (start 165.1508 74.5744) (end 165.1508 75.692) (width 0.25) (layer "B.Cu") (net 4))
 (segment (start 165.1508 75.692) (end 162.4076 78.4352) (width 0.25) (layer "B.Cu") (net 4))
 (segment (start 160.5908 76.0744) (end 160.5908 79.1076) (width 0.25) (layer "F.Cu") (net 5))
 (segment (start 163.040305 77.7102) (end 160.6046 77.7102) (width 0.25) (layer "F.Cu") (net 5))
 (segment (start 160.6046 77.7102) (end 160.5908 77.724) (width 0.25) (layer "F.Cu") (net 5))
 (segment (start 160.5908 79.1076) (end 161.29 79.8068) (width 0.25) (layer "F.Cu") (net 5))
 (segment (start 169.362 70.4944) (end 169.362 71.388505) (width 0.25) (layer "F.Cu") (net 5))
 (segment (start 169.362 71.388505) (end 163.040305 77.7102) (width 0.25) (layer "F.Cu") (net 5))
 (segment (start 164.5372 80.9712) (end 165.1 81.534) (width 0.25) (layer "F.Cu") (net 3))
 (segment (start 164.5372 79.756) (end 164.5372 80.9712) (width 0.25) (layer "F.Cu") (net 3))
 (segment (start 165.7604 69.2404) (end 165.7604 70.4088) (width 0.25) (layer "F.Cu") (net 7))
 (segment (start 165.7604 70.4088) (end 165.2524 70.9168) (width 0.25) (layer "F.Cu") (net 7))
 (segment (start 158.5588 73.8244) (end 158.242 73.5076) (width 0.25) (layer "F.Cu") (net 12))
 (segment (start 159.8408 73.8244) (end 158.5588 73.8244) (width 0.25) (layer "F.Cu") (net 12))
 (segment (start 159.6416 74.5236) (end 159.8408 74.3244) (width 0.25) (layer "F.Cu") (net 2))
 (segment (start 158.242 74.5236) (end 159.6416 74.5236) (width 0.25) (layer "F.Cu") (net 2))
 (segment (start 167.5892 78.7908) (end 166.5732 79.8068) (width 0.25) (layer "F.Cu") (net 2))
 (segment (start 169.3672 78.7908) (end 167.5892 78.7908) (width 0.25) (layer "F.Cu") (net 2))
 (segment (start 167.6908 79.0448) (end 167.64 78.994) (width 0.25) (layer "F.Cu") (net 2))
 (segment (start 159.8408 74.8244) (end 159.8408 74.3244) (width 0.25) (layer "F.Cu") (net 2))
 (via (at 158.242 74.5236) (size 0.8) (drill 0.4) (layers "F.Cu" "B.Cu") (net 2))
 (via (at 166.5732 79.8068) (size 0.8) (drill 0.4) (layers "F.Cu" "B.Cu") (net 2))
 (segment (start 166.5732 79.8068) (end 160.6296 79.8068) (width 0.25) (layer "B.Cu") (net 2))
 (segment (start 160.6296 79.8068) (end 158.242 77.4192) (width 0.25) (layer "B.Cu") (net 2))
 (segment (start 158.242 77.4192) (end 158.242 74.5236) (width 0.25) (layer "B.Cu") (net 2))
 (segment (start 161.5908 76.7744) (end 161.6158 76.7994) (width 0.25) (layer "F.Cu") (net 9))
 (segment (start 162.9258 76.7994) (end 163.576 76.1492) (width 0.25) (layer "F.Cu") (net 9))
 (segment (start 161.5908 76.0744) (end 161.5908 76.7744) (width 0.25) (layer "F.Cu") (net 9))
 (segment (start 161.6158 76.7994) (end 162.9258 76.7994) (width 0.25) (layer "F.Cu") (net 9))
 (segment (start 164.0372 73.152) (end 163.9824 73.152) (width 0.25) (layer "F.Cu") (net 9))
 (segment (start 166.2724 70.9168) (end 164.0372 73.152) (width 0.25) (layer "F.Cu") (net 9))
 (via (at 163.576 76.1492) (size 0.8) (drill 0.4) (layers "F.Cu" "B.Cu") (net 9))
 (via (at 163.9824 73.152) (size 0.8) (drill 0.4) (layers "F.Cu" "B.Cu") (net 9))
 (segment (start 163.5114 73.623) (end 163.9824 73.152) (width 0.25) (layer "B.Cu") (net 9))
 (segment (start 163.5114 76.0846) (end 163.5114 73.623) (width 0.25) (layer "B.Cu") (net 9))
 (segment (start 163.576 76.1492) (end 163.5114 76.0846) (width 0.25) (layer "B.Cu") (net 9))
 (segment (start 162.8408 75.3244) (end 164.1976 75.3244) (width 0.25) (layer "F.Cu") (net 10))
 (segment (start 165.608 79.7052) (end 165.5572 79.756) (width 0.25) (layer "F.Cu") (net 10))
 (segment (start 164.1976 75.3244) (end 164.2364 75.2856) (width 0.25) (layer "F.Cu") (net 10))
 (segment (start 165.608 78.5368) (end 165.608 79.7052) (width 0.25) (layer "F.Cu") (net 10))
 (via (at 165.608 78.5368) (size 0.8) (drill 0.4) (layers "F.Cu" "B.Cu") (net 10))
 (via (at 164.2364 75.2856) (size 0.8) (drill 0.4) (layers "F.Cu" "B.Cu") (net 10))
 (segment (start 165.9128 74.311095) (end 165.9128 78.232) (width 0.25) (layer "B.Cu") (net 10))
 (segment (start 164.2364 74.463495) (end 164.850495 73.8494) (width 0.25) (layer "B.Cu") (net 10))
 (segment (start 165.451105 73.8494) (end 165.9128 74.311095) (width 0.25) (layer "B.Cu") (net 10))
 (segment (start 164.2364 75.2856) (end 164.2364 74.463495) (width 0.25) (layer "B.Cu") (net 10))
 (segment (start 165.9128 78.232) (end 165.608 78.5368) (width 0.25) (layer "B.Cu") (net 10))
 (segment (start 164.850495 73.8494) (end 165.451105 73.8494) (width 0.25) (layer "B.Cu") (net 10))
 (segment (start 162.8408 71.7576) (end 162.8648 71.7336) (width 0.25) (layer "F.Cu") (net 11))
 (segment (start 162.8408 73.8244) (end 162.8408 71.7576) (width 0.25) (layer "F.Cu") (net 11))
 (segment (start 161.0908 71.8312) (end 161.2392 71.6828) (width 0.25) (layer "F.Cu") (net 6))
 (segment (start 161.0908 73.0744) (end 161.0908 71.8312) (width 0.25) (layer "F.Cu") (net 6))
 (segment (start 160.5908 72.2536) (end 160.02 71.6828) (width 0.25) (layer "F.Cu") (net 14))
 (segment (start 160.5908 73.0744) (end 160.5908 72.2536) (width 0.25) (layer "F.Cu") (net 14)))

